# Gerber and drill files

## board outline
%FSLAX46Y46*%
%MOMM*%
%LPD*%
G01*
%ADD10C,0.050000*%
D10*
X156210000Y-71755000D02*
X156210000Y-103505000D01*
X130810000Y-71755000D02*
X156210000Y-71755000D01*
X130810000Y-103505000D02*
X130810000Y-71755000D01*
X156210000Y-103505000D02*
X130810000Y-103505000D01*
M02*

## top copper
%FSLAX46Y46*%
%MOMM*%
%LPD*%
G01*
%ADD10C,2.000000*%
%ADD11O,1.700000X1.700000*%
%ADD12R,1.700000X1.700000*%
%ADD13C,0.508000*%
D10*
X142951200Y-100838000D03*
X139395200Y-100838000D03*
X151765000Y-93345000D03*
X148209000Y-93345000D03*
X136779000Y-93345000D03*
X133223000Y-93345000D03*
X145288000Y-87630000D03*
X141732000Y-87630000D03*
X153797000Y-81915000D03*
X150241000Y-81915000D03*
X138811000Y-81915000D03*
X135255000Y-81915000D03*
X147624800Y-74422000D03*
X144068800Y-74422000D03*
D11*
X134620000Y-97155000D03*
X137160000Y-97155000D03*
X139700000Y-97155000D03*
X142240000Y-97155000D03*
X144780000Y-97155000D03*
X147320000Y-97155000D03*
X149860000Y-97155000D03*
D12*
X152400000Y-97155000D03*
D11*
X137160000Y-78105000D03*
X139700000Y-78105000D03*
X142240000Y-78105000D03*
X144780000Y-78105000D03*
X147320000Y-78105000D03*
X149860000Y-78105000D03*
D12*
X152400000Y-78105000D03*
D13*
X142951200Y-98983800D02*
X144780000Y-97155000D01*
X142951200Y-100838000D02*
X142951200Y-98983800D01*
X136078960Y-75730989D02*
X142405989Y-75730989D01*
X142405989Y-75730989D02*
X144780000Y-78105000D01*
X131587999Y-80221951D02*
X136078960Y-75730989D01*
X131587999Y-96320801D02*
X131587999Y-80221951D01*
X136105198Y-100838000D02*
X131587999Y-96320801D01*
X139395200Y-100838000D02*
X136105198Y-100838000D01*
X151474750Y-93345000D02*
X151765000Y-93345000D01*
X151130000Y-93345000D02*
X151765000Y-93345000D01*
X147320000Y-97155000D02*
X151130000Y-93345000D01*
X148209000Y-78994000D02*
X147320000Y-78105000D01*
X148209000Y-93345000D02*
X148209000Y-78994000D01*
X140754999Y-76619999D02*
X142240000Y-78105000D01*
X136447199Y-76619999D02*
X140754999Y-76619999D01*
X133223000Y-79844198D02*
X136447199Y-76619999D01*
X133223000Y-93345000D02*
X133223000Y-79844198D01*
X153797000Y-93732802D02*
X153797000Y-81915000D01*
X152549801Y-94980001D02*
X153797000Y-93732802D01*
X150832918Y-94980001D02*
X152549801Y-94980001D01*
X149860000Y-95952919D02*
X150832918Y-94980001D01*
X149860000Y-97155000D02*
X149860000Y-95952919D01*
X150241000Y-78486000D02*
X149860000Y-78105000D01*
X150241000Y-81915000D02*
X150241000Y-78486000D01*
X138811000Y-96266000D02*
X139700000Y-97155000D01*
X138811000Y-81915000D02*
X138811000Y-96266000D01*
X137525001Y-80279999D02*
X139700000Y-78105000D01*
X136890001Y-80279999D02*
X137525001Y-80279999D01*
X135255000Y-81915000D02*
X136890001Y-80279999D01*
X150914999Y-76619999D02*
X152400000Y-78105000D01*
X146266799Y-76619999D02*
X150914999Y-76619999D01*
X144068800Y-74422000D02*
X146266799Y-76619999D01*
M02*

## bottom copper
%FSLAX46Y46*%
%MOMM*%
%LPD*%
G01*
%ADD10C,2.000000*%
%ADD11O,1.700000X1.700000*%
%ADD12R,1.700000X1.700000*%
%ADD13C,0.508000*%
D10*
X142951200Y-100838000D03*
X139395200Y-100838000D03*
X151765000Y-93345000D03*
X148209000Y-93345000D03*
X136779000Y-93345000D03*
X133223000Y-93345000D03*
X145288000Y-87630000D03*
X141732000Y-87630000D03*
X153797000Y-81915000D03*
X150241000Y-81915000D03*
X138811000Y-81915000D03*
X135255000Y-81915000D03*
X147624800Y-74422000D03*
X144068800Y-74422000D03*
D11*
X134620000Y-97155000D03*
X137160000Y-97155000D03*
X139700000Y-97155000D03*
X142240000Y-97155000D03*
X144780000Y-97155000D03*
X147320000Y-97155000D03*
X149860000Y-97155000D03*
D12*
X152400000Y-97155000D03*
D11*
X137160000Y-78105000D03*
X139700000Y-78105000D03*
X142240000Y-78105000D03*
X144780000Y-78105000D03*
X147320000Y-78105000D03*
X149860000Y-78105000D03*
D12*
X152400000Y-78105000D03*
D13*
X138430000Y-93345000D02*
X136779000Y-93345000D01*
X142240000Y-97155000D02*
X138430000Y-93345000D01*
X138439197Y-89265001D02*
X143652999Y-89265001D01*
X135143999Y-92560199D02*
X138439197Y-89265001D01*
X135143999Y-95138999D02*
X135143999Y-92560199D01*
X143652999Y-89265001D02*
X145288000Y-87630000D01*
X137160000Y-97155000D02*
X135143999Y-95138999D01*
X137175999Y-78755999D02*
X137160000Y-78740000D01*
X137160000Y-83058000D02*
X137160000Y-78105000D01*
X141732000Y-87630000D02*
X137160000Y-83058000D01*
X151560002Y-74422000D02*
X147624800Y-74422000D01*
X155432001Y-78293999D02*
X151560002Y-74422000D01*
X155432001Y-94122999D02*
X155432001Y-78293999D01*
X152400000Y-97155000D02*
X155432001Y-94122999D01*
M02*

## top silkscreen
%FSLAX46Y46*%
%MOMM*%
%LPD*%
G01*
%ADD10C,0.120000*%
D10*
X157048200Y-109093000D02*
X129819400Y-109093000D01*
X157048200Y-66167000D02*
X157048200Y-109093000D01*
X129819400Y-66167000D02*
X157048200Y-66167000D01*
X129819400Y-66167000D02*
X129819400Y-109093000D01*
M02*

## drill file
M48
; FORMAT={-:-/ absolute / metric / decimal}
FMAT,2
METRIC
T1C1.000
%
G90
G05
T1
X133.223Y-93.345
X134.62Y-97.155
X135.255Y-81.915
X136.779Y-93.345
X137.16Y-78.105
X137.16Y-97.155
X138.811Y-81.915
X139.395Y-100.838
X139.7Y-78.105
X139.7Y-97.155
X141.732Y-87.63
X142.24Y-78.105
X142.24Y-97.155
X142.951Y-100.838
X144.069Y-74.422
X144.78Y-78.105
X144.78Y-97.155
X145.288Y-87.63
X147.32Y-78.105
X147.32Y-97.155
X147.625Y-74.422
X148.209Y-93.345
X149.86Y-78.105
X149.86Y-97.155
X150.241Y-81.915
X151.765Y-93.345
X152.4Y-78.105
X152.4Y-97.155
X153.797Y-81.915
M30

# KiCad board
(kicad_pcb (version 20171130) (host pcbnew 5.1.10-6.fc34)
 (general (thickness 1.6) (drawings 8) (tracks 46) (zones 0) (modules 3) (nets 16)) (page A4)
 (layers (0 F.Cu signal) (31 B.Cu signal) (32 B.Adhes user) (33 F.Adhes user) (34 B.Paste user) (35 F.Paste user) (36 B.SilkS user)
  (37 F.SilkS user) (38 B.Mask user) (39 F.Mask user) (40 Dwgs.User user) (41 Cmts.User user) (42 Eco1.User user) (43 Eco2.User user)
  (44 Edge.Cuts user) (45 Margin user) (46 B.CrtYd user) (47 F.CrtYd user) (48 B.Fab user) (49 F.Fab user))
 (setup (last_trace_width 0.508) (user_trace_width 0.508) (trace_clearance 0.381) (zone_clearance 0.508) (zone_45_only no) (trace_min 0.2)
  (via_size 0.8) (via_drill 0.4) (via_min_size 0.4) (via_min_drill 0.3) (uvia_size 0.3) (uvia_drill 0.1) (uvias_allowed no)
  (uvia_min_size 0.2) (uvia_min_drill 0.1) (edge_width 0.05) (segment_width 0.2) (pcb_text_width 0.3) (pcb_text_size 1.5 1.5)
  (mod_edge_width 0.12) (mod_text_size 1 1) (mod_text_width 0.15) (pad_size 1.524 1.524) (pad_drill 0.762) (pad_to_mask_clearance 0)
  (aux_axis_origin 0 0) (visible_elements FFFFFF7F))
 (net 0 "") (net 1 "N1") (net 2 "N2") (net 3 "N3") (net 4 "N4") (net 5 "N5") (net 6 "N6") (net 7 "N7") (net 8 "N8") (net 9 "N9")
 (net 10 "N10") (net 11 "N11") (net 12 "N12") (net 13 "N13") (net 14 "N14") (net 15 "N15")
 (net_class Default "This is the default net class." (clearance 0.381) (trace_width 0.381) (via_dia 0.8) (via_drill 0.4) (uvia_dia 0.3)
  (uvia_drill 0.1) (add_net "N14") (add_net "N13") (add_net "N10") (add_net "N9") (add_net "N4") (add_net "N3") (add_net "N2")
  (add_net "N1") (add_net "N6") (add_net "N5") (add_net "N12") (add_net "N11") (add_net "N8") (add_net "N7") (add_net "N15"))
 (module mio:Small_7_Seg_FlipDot (layer F.Cu) (at 143.51 87.63)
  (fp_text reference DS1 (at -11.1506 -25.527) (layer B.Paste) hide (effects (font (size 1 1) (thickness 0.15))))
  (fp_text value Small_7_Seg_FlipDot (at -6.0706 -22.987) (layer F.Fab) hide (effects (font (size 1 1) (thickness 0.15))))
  (fp_line (start 13.5382 21.463) (end -13.6906 21.463) (layer F.SilkS) (width 0.12))
  (fp_line (start 13.5382 -21.463) (end 13.5382 21.463) (layer F.SilkS) (width 0.12))
  (fp_line (start -13.6906 -21.463) (end 13.5382 -21.463) (layer F.SilkS) (width 0.12))
  (fp_line (start -13.6906 -21.463) (end -13.6906 21.463) (layer F.SilkS) (width 0.12))
  (pad D2 thru_hole circle (at -0.5588 13.208) (size 2 2) (drill 1) (layers *.Cu *.Mask) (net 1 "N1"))
  (pad D1 thru_hole circle (at -4.1148 13.208) (size 2 2) (drill 1) (layers *.Cu *.Mask) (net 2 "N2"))
  (pad C2 thru_hole circle (at 8.255 5.715) (size 2 2) (drill 1) (layers *.Cu *.Mask) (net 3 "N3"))
  (pad C1 thru_hole circle (at 4.699 5.715) (size 2 2) (drill 1) (layers *.Cu *.Mask) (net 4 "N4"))
  (pad E2 thru_hole circle (at -6.731 5.715) (size 2 2) (drill 1) (layers *.Cu *.Mask) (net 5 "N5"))
  (pad E1 thru_hole circle (at -10.287 5.715) (size 2 2) (drill 1) (layers *.Cu *.Mask) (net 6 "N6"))
  (pad G2 thru_hole circle (at 1.778 0) (size 2 2) (drill 1) (layers *.Cu *.Mask) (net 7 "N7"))
  (pad G1 thru_hole circle (at -1.778 0) (size 2 2) (drill 1) (layers *.Cu *.Mask) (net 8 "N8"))
  (pad B2 thru_hole circle (at 10.287 -5.715) (size 2 2) (drill 1) (layers *.Cu *.Mask) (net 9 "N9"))
  (pad B1 thru_hole circle (at 6.731 -5.715) (size 2 2) (drill 1) (layers *.Cu *.Mask) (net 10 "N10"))
  (pad F2 thru_hole circle (at -4.699 -5.715) (size 2 2) (drill 1) (layers *.Cu *.Mask) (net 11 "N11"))
  (pad F1 thru_hole circle (at -8.255 -5.715) (size 2 2) (drill 1) (layers *.Cu *.Mask) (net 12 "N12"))
  (pad A2 thru_hole circle (at 4.1148 -13.208) (size 2 2) (drill 1) (layers *.Cu *.Mask) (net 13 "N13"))
  (pad A1 thru_hole circle (at 0.5588 -13.208) (size 2 2) (drill 1) (layers *.Cu *.Mask) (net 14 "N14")))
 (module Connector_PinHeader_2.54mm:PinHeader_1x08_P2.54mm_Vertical (layer B.Cu) (at 152.4 97.155 90)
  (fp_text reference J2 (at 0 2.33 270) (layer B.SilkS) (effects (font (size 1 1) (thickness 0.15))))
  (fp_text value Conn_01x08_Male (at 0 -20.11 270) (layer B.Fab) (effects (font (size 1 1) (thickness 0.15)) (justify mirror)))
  (pad 8 thru_hole oval (at 0 -17.78 90) (size 1.7 1.7) (drill 1) (layers *.Cu *.Mask) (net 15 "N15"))
  (pad 7 thru_hole oval (at 0 -15.24 90) (size 1.7 1.7) (drill 1) (layers *.Cu *.Mask) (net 7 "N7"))
  (pad 6 thru_hole oval (at 0 -12.7 90) (size 1.7 1.7) (drill 1) (layers *.Cu *.Mask) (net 11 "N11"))
  (pad 5 thru_hole oval (at 0 -10.16 90) (size 1.7 1.7) (drill 1) (layers *.Cu *.Mask) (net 5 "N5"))
  (pad 4 thru_hole oval (at 0 -7.62 90) (size 1.7 1.7) (drill 1) (layers *.Cu *.Mask) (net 1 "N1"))
  (pad 3 thru_hole oval (at 0 -5.08 90) (size 1.7 1.7) (drill 1) (layers *.Cu *.Mask) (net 3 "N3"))
  (pad 2 thru_hole oval (at 0 -2.54 90) (size 1.7 1.7) (drill 1) (layers *.Cu *.Mask) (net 9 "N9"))
  (pad 1 thru_hole rect (at 0 0 90) (size 1.7 1.7) (drill 1) (layers *.Cu *.Mask) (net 13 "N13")))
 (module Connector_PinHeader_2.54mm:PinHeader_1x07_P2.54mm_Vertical (layer B.Cu) (at 152.4 78.105 90)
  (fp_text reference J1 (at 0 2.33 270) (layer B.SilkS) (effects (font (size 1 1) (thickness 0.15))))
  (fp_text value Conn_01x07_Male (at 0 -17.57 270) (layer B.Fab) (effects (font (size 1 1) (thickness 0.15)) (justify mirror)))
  (pad 7 thru_hole oval (at 0 -15.24 90) (size 1.7 1.7) (drill 1) (layers *.Cu *.Mask) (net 8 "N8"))
  (pad 6 thru_hole oval (at 0 -12.7 90) (size 1.7 1.7) (drill 1) (layers *.Cu *.Mask) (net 12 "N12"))
  (pad 5 thru_hole oval (at 0 -10.16 90) (size 1.7 1.7) (drill 1) (layers *.Cu *.Mask) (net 6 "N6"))
  (pad 4 thru_hole oval (at 0 -7.62 90) (size 1.7 1.7) (drill 1) (layers *.Cu *.Mask) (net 2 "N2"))
  (pad 3 thru_hole oval (at 0 -5.08 90) (size 1.7 1.7) (drill 1) (layers *.Cu *.Mask) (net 4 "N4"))
  (pad 2 thru_hole oval (at 0 -2.54 90) (size 1.7 1.7) (drill 1) (layers *.Cu *.Mask) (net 10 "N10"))
  (pad 1 thru_hole rect (at 0 0 90) (size 1.7 1.7) (drill 1) (layers *.Cu *.Mask) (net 14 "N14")))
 (gr_line (start 156.21 71.755) (end 156.21 103.505) (layer Edge.Cuts) (width 0.05))
 (gr_line (start 130.81 71.755) (end 156.21 71.755) (layer Edge.Cuts) (width 0.05))
 (gr_line (start 130.81 103.505) (end 130.81 71.755) (layer Edge.Cuts) (width 0.05))
 (gr_line (start 156.21 103.505) (end 130.81 103.505) (layer Edge.Cuts) (width 0.05))
 (segment (start 142.9512 98.9838) (end 144.78 97.155) (width 0.508) (layer F.Cu) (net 1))
 (segment (start 142.9512 100.838) (end 142.9512 98.9838) (width 0.508) (layer F.Cu) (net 1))
 (segment (start 136.07896 75.730989) (end 142.405989 75.730989) (width 0.508) (layer F.Cu) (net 2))
 (segment (start 142.405989 75.730989) (end 144.78 78.105) (width 0.508) (layer F.Cu) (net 2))
 (segment (start 131.587999 80.221951) (end 136.07896 75.730989) (width 0.508) (layer F.Cu) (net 2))
 (segment (start 131.587999 96.320801) (end 131.587999 80.221951) (width 0.508) (layer F.Cu) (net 2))
 (segment (start 136.105198 100.838) (end 131.587999 96.320801) (width 0.508) (layer F.Cu) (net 2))
 (segment (start 139.3952 100.838) (end 136.105198 100.838) (width 0.508) (layer F.Cu) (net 2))
 (segment (start 151.47475 93.345) (end 151.765 93.345) (width 0.508) (layer F.Cu) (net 3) (status 30))
 (segment (start 151.13 93.345) (end 151.765 93.345) (width 0.508) (layer F.Cu) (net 3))
 (segment (start 147.32 97.155) (end 151.13 93.345) (width 0.508) (layer F.Cu) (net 3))
 (segment (start 148.209 78.994) (end 147.32 78.105) (width 0.508) (layer F.Cu) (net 4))
 (segment (start 148.209 93.345) (end 148.209 78.994) (width 0.508) (layer F.Cu) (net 4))
 (segment (start 138.43 93.345) (end 136.779 93.345) (width 0.508) (layer B.Cu) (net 5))
 (segment (start 142.24 97.155) (end 138.43 93.345) (width 0.508) (layer B.Cu) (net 5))
 (segment (start 140.754999 76.619999) (end 142.24 78.105) (width 0.508) (layer F.Cu) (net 6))
 (segment (start 136.447199 76.619999) (end 140.754999 76.619999) (width 0.508) (layer F.Cu) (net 6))
 (segment (start 133.223 79.844198) (end 136.447199 76.619999) (width 0.508) (layer F.Cu) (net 6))
 (segment (start 133.223 93.345) (end 133.223 79.844198) (width 0.508) (layer F.Cu) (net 6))
 (segment (start 138.439197 89.265001) (end 143.652999 89.265001) (width 0.508) (layer B.Cu) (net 7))
 (segment (start 135.143999 92.560199) (end 138.439197 89.265001) (width 0.508) (layer B.Cu) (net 7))
 (segment (start 135.143999 95.138999) (end 135.143999 92.560199) (width 0.508) (layer B.Cu) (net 7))
 (segment (start 143.652999 89.265001) (end 145.288 87.63) (width 0.508) (layer B.Cu) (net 7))
 (segment (start 137.16 97.155) (end 135.143999 95.138999) (width 0.508) (layer B.Cu) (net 7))
 (segment (start 137.175999 78.755999) (end 137.16 78.74) (width 0.508) (layer B.Cu) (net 8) (status 30))
 (segment (start 137.16 83.058) (end 137.16 78.105) (width 0.508) (layer B.Cu) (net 8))
 (segment (start 141.732 87.63) (end 137.16 83.058) (width 0.508) (layer B.Cu) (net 8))
 (segment (start 153.797 93.732802) (end 153.797 81.915) (width 0.508) (layer F.Cu) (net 9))
 (segment (start 152.549801 94.980001) (end 153.797 93.732802) (width 0.508) (layer F.Cu) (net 9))
 (segment (start 150.832918 94.980001) (end 152.549801 94.980001) (width 0.508) (layer F.Cu) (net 9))
 (segment (start 149.86 95.952919) (end 150.832918 94.980001) (width 0.508) (layer F.Cu) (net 9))
 (segment (start 149.86 97.155) (end 149.86 95.952919) (width 0.508) (layer F.Cu) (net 9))
 (segment (start 150.241 78.486) (end 149.86 78.105) (width 0.508) (layer F.Cu) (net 10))
 (segment (start 150.241 81.915) (end 150.241 78.486) (width 0.508) (layer F.Cu) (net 10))
 (segment (start 138.811 96.266) (end 139.7 97.155) (width 0.508) (layer F.Cu) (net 11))
 (segment (start 138.811 81.915) (end 138.811 96.266) (width 0.508) (layer F.Cu) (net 11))
 (segment (start 137.525001 80.279999) (end 139.7 78.105) (width 0.508) (layer F.Cu) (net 12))
 (segment (start 136.890001 80.279999) (end 137.525001 80.279999) (width 0.508) (layer F.Cu) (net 12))
 (segment (start 135.255 81.915) (end 136.890001 80.279999) (width 0.508) (layer F.Cu) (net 12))
 (segment (start 151.560002 74.422) (end 147.6248 74.422) (width 0.508) (layer B.Cu) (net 13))
 (segment (start 155.432001 78.293999) (end 151.560002 74.422) (width 0.508) (layer B.Cu) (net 13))
 (segment (start 155.432001 94.122999) (end 155.432001 78.293999) (width 0.508) (layer B.Cu) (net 13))
 (segment (start 152.4 97.155) (end 155.432001 94.122999) (width 0.508) (layer B.Cu) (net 13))
 (segment (start 150.914999 76.619999) (end 152.4 78.105) (width 0.508) (layer F.Cu) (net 14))
 (segment (start 146.266799 76.619999) (end 150.914999 76.619999) (width 0.508) (layer F.Cu) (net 14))
 (segment (start 144.0688 74.422) (end 146.266799 76.619999) (width 0.508) (layer F.Cu) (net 14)))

